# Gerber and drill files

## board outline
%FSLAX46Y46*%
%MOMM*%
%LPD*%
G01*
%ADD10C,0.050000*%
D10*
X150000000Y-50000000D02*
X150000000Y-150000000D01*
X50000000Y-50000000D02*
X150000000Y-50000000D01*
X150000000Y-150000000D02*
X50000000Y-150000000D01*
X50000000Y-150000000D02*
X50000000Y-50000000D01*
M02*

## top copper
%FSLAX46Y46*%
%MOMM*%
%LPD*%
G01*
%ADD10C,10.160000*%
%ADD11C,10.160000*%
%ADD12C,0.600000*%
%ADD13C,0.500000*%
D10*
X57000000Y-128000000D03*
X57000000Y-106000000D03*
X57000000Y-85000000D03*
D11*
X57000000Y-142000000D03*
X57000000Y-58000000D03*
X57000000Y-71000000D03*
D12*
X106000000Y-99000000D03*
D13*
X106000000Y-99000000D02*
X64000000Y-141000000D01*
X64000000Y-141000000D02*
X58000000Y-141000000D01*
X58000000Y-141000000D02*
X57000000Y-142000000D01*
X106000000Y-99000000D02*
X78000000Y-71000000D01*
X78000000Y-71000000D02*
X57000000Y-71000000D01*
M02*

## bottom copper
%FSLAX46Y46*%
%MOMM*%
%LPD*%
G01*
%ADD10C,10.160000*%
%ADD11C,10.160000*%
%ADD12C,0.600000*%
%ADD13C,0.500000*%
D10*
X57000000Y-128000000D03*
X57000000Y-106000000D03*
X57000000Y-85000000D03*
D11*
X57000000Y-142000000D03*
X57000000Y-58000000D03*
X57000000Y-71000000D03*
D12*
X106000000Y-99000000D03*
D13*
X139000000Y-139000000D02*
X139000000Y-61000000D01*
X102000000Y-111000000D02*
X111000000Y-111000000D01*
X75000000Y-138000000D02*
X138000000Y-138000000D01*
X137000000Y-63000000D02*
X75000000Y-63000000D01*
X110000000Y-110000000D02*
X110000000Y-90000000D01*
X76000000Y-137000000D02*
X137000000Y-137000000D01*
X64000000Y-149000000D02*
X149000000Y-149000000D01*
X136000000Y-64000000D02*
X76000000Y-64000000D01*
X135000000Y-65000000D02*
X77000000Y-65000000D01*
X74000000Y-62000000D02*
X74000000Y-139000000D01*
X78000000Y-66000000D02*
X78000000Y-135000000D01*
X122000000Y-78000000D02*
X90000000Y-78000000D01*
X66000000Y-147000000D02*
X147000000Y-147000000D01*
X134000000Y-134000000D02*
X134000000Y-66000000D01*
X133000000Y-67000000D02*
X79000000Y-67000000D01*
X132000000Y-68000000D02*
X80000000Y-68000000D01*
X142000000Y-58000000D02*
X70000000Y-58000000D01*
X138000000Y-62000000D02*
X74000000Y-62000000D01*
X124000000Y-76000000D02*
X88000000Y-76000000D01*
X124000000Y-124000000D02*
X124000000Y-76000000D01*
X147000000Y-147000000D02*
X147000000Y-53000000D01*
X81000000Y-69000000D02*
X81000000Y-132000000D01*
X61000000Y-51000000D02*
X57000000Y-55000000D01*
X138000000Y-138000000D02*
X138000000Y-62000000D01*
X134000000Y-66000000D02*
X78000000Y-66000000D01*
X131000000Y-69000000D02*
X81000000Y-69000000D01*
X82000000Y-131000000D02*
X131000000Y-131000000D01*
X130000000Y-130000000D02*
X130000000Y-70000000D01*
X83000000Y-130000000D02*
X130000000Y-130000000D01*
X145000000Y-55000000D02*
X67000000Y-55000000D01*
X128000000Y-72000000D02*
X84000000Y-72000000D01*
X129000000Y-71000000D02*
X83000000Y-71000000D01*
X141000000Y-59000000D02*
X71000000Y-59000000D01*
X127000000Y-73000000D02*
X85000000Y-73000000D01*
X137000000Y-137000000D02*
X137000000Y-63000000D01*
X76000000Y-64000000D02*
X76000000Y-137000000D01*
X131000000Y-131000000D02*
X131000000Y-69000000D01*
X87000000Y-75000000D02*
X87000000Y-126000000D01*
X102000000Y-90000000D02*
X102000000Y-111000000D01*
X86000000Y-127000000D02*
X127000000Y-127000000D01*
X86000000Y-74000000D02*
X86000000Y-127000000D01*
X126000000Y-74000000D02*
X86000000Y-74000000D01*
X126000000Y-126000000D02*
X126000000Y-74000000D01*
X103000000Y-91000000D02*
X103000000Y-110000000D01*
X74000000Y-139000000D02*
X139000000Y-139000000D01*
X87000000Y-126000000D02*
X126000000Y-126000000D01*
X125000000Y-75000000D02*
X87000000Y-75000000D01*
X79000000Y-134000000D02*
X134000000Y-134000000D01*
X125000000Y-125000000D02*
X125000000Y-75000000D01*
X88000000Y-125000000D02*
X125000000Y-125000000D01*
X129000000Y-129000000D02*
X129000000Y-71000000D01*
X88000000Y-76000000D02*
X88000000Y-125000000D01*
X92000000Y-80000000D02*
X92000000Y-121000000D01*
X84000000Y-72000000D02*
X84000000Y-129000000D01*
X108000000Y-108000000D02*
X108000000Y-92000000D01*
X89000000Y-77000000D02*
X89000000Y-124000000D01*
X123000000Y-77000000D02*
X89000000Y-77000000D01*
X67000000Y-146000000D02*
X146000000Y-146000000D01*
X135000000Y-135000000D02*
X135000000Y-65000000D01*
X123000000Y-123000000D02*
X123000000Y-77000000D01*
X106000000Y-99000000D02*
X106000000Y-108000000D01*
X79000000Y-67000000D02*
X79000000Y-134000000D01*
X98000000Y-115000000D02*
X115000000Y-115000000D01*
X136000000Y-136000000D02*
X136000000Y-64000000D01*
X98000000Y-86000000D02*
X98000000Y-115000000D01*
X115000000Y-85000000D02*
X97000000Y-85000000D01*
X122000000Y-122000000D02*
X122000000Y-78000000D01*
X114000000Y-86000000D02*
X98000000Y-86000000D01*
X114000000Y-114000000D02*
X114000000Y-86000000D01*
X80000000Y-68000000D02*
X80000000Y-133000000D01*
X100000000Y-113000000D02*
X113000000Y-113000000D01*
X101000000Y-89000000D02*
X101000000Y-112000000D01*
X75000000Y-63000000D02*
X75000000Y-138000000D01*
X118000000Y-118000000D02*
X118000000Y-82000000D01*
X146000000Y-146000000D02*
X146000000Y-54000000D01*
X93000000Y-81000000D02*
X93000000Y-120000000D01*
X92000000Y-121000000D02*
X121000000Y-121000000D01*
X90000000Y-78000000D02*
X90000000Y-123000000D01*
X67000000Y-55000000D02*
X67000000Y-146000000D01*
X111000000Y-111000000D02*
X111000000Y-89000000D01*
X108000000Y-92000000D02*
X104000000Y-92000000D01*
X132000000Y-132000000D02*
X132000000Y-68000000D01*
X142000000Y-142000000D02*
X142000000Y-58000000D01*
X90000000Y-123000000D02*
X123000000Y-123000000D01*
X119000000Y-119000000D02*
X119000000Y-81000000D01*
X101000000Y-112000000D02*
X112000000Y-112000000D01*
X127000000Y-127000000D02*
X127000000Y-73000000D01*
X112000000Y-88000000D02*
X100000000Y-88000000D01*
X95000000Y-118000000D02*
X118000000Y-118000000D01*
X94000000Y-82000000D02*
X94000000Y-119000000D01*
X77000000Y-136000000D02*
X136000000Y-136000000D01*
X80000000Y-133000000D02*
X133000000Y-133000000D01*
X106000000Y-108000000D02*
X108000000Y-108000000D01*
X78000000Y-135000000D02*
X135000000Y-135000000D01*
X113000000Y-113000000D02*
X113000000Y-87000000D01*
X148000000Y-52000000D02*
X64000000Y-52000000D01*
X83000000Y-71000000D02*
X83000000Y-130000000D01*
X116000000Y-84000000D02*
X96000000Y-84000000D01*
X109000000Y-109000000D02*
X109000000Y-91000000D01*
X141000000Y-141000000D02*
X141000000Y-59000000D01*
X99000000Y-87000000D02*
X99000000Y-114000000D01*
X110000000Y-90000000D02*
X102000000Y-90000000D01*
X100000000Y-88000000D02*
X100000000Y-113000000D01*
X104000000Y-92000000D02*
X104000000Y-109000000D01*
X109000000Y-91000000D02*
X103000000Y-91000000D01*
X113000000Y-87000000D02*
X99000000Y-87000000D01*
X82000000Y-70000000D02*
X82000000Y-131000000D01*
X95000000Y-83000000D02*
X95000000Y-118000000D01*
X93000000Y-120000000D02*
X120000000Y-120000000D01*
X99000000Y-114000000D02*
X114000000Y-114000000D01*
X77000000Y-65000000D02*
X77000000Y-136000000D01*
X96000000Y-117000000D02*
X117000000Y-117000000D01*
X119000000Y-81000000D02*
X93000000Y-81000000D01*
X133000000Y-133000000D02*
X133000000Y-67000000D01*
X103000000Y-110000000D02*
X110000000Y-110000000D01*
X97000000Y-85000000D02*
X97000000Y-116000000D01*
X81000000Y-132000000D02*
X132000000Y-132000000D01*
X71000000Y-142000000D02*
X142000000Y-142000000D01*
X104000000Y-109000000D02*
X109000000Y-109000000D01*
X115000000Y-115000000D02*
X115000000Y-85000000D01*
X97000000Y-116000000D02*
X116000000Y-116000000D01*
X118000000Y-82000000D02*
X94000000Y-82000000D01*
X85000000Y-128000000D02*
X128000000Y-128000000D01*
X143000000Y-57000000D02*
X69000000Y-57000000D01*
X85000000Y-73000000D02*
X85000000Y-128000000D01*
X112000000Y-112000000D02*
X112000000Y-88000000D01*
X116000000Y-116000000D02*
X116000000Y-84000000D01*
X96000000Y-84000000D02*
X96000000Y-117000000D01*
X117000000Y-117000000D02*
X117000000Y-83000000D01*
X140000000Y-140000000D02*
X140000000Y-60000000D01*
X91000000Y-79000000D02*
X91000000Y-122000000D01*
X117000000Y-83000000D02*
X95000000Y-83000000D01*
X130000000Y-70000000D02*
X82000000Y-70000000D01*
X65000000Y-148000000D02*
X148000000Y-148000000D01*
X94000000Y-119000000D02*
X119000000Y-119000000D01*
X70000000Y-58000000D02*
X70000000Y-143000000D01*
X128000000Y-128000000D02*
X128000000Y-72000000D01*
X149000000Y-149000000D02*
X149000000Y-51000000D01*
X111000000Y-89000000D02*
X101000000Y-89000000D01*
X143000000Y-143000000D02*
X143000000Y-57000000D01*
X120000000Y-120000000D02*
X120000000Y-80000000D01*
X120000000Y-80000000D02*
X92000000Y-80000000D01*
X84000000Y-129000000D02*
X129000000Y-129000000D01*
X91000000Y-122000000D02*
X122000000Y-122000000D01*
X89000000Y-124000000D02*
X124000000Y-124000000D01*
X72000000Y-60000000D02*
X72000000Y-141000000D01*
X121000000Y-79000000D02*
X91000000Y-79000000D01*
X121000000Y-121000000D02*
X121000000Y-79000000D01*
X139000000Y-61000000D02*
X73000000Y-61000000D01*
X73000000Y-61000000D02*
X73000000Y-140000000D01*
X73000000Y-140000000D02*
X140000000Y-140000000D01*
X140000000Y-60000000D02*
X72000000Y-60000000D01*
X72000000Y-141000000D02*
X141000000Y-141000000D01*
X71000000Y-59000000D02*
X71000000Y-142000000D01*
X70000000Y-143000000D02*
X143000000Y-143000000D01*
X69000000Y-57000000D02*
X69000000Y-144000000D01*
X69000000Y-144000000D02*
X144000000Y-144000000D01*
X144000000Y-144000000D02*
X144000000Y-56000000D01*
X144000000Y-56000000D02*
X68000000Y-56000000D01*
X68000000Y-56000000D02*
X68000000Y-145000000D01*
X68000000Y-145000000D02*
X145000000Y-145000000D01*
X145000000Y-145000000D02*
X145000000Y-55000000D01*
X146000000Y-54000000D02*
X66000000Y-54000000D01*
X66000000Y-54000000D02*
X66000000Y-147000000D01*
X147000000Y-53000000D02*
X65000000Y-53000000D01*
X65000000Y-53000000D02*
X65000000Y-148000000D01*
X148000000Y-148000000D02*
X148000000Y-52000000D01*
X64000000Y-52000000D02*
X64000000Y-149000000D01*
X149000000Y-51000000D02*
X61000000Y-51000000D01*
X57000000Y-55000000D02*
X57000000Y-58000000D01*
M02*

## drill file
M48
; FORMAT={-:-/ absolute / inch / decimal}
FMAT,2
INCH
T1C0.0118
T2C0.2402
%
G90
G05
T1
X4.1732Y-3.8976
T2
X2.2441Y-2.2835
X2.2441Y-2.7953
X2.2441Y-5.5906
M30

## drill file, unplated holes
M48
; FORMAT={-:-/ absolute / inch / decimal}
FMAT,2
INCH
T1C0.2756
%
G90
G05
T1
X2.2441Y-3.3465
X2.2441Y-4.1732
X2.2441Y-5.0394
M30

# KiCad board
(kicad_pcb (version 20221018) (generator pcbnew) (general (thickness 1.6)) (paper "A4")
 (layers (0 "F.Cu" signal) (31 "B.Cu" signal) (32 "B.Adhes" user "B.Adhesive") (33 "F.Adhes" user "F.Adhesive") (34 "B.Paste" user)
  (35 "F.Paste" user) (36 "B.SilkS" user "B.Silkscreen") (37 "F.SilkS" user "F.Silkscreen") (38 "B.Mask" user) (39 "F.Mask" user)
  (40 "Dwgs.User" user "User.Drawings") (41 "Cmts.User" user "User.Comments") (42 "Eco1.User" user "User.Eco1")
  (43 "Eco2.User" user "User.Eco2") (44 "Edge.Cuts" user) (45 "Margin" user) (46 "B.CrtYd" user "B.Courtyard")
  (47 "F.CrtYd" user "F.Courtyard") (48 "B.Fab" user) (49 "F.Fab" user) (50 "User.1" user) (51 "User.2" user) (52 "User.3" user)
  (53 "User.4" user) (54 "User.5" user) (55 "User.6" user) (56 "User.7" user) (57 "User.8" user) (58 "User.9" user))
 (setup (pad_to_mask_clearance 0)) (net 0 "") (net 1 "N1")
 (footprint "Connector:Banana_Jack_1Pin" (layer "F.Cu") (at 57 128)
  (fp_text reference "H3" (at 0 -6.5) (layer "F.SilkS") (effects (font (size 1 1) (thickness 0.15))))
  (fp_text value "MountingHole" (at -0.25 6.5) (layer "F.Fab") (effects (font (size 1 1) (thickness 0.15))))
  (pad "" np_thru_hole circle (at 0 0) (size 10.16 10.16) (drill 7) (layers "F&B.Cu" "*.Mask")))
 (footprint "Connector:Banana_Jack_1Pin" (layer "F.Cu") (at 57 58)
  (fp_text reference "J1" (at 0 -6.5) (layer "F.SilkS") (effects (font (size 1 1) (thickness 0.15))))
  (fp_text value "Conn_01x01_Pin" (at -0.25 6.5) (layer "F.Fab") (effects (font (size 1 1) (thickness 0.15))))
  (pad "1" thru_hole circle (at 0 0) (size 10.16 10.16) (drill 6.1) (layers "*.Cu" "*.Mask") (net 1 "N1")))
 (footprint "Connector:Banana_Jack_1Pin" (layer "F.Cu") (at 57 71)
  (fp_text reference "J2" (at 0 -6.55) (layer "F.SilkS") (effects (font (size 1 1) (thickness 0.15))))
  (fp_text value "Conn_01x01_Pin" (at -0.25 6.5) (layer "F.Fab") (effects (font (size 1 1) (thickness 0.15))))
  (pad "1" thru_hole circle (at 0 0) (size 10.16 10.16) (drill 6.1) (layers "*.Cu" "*.Mask") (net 1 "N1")))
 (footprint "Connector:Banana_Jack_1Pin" (layer "F.Cu") (at 57 106)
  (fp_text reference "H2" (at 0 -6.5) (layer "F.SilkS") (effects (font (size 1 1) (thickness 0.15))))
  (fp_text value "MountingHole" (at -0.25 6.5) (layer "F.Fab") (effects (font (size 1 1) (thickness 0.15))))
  (pad "" np_thru_hole circle (at 0 0) (size 10.16 10.16) (drill 7) (layers "F&B.Cu" "*.Mask")))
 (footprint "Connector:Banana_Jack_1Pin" (layer "F.Cu") (at 57 142)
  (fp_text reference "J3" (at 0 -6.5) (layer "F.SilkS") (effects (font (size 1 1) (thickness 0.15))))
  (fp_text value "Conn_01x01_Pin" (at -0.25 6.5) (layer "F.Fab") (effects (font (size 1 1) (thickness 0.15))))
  (pad "1" thru_hole circle (at 0 0) (size 10.16 10.16) (drill 6.1) (layers "*.Cu" "*.Mask") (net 1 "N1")))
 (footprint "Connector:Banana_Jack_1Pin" (layer "F.Cu") (at 57 85)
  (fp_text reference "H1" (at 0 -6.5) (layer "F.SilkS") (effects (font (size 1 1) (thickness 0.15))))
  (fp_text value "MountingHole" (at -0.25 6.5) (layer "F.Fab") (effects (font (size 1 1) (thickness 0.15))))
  (pad "" np_thru_hole circle (at 0 0) (size 10.16 10.16) (drill 7) (layers "F&B.Cu" "*.Mask")))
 (gr_line (start 150 50) (end 150 150) (stroke (width 0.05) (type default)) (layer "Edge.Cuts"))
 (gr_line (start 50 50) (end 150 50) (stroke (width 0.05) (type default)) (layer "Edge.Cuts"))
 (gr_line (start 150 150) (end 50 150) (stroke (width 0.05) (type default)) (layer "Edge.Cuts"))
 (gr_line (start 50 150) (end 50 50) (stroke (width 0.05) (type default)) (layer "Edge.Cuts"))
 (segment (start 106 99) (end 64 141) (width 0.5) (layer "F.Cu") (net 1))
 (segment (start 106 99) (end 78 71) (width 0.5) (layer "F.Cu") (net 1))
 (segment (start 64 141) (end 58 141) (width 0.5) (layer "F.Cu") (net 1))
 (segment (start 58 141) (end 57 142) (width 0.5) (layer "F.Cu") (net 1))
 (segment (start 78 71) (end 57 71) (width 0.5) (layer "F.Cu") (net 1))
 (via (at 106 99) (size 0.6) (drill 0.3) (layers "F.Cu" "B.Cu") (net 1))
 (segment (start 121 79) (end 91 79) (width 0.5) (layer "B.Cu") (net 1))
 (segment (start 82 131) (end 131 131) (width 0.5) (layer "B.Cu") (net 1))
 (segment (start 124 124) (end 124 76) (width 0.5) (layer "B.Cu") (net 1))
 (segment (start 83 71) (end 83 130) (width 0.5) (layer "B.Cu") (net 1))
 (segment (start 89 77) (end 89 124) (width 0.5) (layer "B.Cu") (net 1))
 (segment (start 100 113) (end 113 113) (width 0.5) (layer "B.Cu") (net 1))
 (segment (start 120 120) (end 120 80) (width 0.5) (layer "B.Cu") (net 1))
 (segment (start 67 146) (end 146 146) (width 0.5) (layer "B.Cu") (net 1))
 (segment (start 66 54) (end 66 147) (width 0.5) (layer "B.Cu") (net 1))
 (segment (start 92 80) (end 92 121) (width 0.5) (layer "B.Cu") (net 1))
 (segment (start 98 86) (end 98 115) (width 0.5) (layer "B.Cu") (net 1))
 (segment (start 90 123) (end 123 123) (width 0.5) (layer "B.Cu") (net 1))
 (segment (start 146 54) (end 66 54) (width 0.5) (layer "B.Cu") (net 1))
 (segment (start 120 80) (end 92 80) (width 0.5) (layer "B.Cu") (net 1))
 (segment (start 76 137) (end 137 137) (width 0.5) (layer "B.Cu") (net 1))
 (segment (start 92 121) (end 121 121) (width 0.5) (layer "B.Cu") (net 1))
 (segment (start 121 121) (end 121 79) (width 0.5) (layer "B.Cu") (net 1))
 (segment (start 112 88) (end 100 88) (width 0.5) (layer "B.Cu") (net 1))
 (segment (start 135 65) (end 77 65) (width 0.5) (layer "B.Cu") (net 1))
 (segment (start 68 145) (end 145 145) (width 0.5) (layer "B.Cu") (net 1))
 (segment (start 86 127) (end 127 127) (width 0.5) (layer "B.Cu") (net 1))
 (segment (start 73 140) (end 140 140) (width 0.5) (layer "B.Cu") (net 1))
 (segment (start 114 86) (end 98 86) (width 0.5) (layer "B.Cu") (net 1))
 (segment (start 96 117) (end 117 117) (width 0.5) (layer "B.Cu") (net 1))
 (segment (start 57 55) (end 57 58) (width 0.5) (layer "B.Cu") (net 1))
 (segment (start 95 118) (end 118 118) (width 0.5) (layer "B.Cu") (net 1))
 (segment (start 80 68) (end 80 133) (width 0.5) (layer "B.Cu") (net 1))
 (segment (start 83 130) (end 130 130) (width 0.5) (layer "B.Cu") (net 1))
 (segment (start 148 52) (end 64 52) (width 0.5) (layer "B.Cu") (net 1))
 (segment (start 145 145) (end 145 55) (width 0.5) (layer "B.Cu") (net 1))
 (segment (start 129 129) (end 129 71) (width 0.5) (layer "B.Cu") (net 1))
 (segment (start 68 56) (end 68 145) (width 0.5) (layer "B.Cu") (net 1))
 (segment (start 127 127) (end 127 73) (width 0.5) (layer "B.Cu") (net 1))
 (segment (start 109 91) (end 103 91) (width 0.5) (layer "B.Cu") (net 1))
 (segment (start 84 72) (end 84 129) (width 0.5) (layer "B.Cu") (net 1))
 (segment (start 71 59) (end 71 142) (width 0.5) (layer "B.Cu") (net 1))
 (segment (start 85 73) (end 85 128) (width 0.5) (layer "B.Cu") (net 1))
 (segment (start 102 90) (end 102 111) (width 0.5) (layer "B.Cu") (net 1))
 (segment (start 72 60) (end 72 141) (width 0.5) (layer "B.Cu") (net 1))
 (segment (start 142 142) (end 142 58) (width 0.5) (layer "B.Cu") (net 1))
 (segment (start 131 131) (end 131 69) (width 0.5) (layer "B.Cu") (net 1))
 (segment (start 65 148) (end 148 148) (width 0.5) (layer "B.Cu") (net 1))
 (segment (start 71 142) (end 142 142) (width 0.5) (layer "B.Cu") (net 1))
 (segment (start 101 89) (end 101 112) (width 0.5) (layer "B.Cu") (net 1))
 (segment (start 99 114) (end 114 114) (width 0.5) (layer "B.Cu") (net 1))
 (segment (start 149 51) (end 61 51) (width 0.5) (layer "B.Cu") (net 1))
 (segment (start 128 128) (end 128 72) (width 0.5) (layer "B.Cu") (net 1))
 (segment (start 72 141) (end 141 141) (width 0.5) (layer "B.Cu") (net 1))
 (segment (start 66 147) (end 147 147) (width 0.5) (layer "B.Cu") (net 1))
 (segment (start 126 74) (end 86 74) (width 0.5) (layer "B.Cu") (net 1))
 (segment (start 102 111) (end 111 111) (width 0.5) (layer "B.Cu") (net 1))
 (segment (start 87 126) (end 126 126) (width 0.5) (layer "B.Cu") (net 1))
 (segment (start 119 119) (end 119 81) (width 0.5) (layer "B.Cu") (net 1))
 (segment (start 133 67) (end 79 67) (width 0.5) (layer "B.Cu") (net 1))
 (segment (start 94 119) (end 119 119) (width 0.5) (layer "B.Cu") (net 1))
 (segment (start 90 78) (end 90 123) (width 0.5) (layer "B.Cu") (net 1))
 (segment (start 147 147) (end 147 53) (width 0.5) (layer "B.Cu") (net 1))
 (segment (start 146 146) (end 146 54) (width 0.5) (layer "B.Cu") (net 1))
 (segment (start 111 111) (end 111 89) (width 0.5) (layer "B.Cu") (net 1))
 (segment (start 74 62) (end 74 139) (width 0.5) (layer "B.Cu") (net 1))
 (segment (start 148 148) (end 148 52) (width 0.5) (layer "B.Cu") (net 1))
 (segment (start 147 53) (end 65 53) (width 0.5) (layer "B.Cu") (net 1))
 (segment (start 132 68) (end 80 68) (width 0.5) (layer "B.Cu") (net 1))
 (segment (start 79 67) (end 79 134) (width 0.5) (layer "B.Cu") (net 1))
 (segment (start 74 139) (end 139 139) (width 0.5) (layer "B.Cu") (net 1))
 (segment (start 125 125) (end 125 75) (width 0.5) (layer "B.Cu") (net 1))
 (segment (start 104 92) (end 104 109) (width 0.5) (layer "B.Cu") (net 1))
 (segment (start 125 75) (end 87 75) (width 0.5) (layer "B.Cu") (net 1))
 (segment (start 136 136) (end 136 64) (width 0.5) (layer "B.Cu") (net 1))
 (segment (start 61 51) (end 57 55) (width 0.5) (layer "B.Cu") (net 1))
 (segment (start 145 55) (end 67 55) (width 0.5) (layer "B.Cu") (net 1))
 (segment (start 113 87) (end 99 87) (width 0.5) (layer "B.Cu") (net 1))
 (segment (start 89 124) (end 124 124) (width 0.5) (layer "B.Cu") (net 1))
 (segment (start 129 71) (end 83 71) (width 0.5) (layer "B.Cu") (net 1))
 (segment (start 114 114) (end 114 86) (width 0.5) (layer "B.Cu") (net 1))
 (segment (start 85 128) (end 128 128) (width 0.5) (layer "B.Cu") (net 1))
 (segment (start 144 144) (end 144 56) (width 0.5) (layer "B.Cu") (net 1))
 (segment (start 97 116) (end 116 116) (width 0.5) (layer "B.Cu") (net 1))
 (segment (start 64 149) (end 149 149) (width 0.5) (layer "B.Cu") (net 1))
 (segment (start 139 61) (end 73 61) (width 0.5) (layer "B.Cu") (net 1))
 (segment (start 86 74) (end 86 127) (width 0.5) (layer "B.Cu") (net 1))
 (segment (start 93 81) (end 93 120) (width 0.5) (layer "B.Cu") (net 1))
 (segment (start 138 138) (end 138 62) (width 0.5) (layer "B.Cu") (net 1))
 (segment (start 118 118) (end 118 82) (width 0.5) (layer "B.Cu") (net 1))
 (segment (start 140 140) (end 140 60) (width 0.5) (layer "B.Cu") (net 1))
 (segment (start 106 99) (end 106 108) (width 0.5) (layer "B.Cu") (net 1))
 (segment (start 78 66) (end 78 135) (width 0.5) (layer "B.Cu") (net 1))
 (segment (start 138 62) (end 74 62) (width 0.5) (layer "B.Cu") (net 1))
 (segment (start 118 82) (end 94 82) (width 0.5) (layer "B.Cu") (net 1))
 (segment (start 110 90) (end 102 90) (width 0.5) (layer "B.Cu") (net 1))
 (segment (start 132 132) (end 132 68) (width 0.5) (layer "B.Cu") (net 1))
 (segment (start 78 135) (end 135 135) (width 0.5) (layer "B.Cu") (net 1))
 (segment (start 136 64) (end 76 64) (width 0.5) (layer "B.Cu") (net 1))
 (segment (start 75 63) (end 75 138) (width 0.5) (layer "B.Cu") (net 1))
 (segment (start 123 77) (end 89 77) (width 0.5) (layer "B.Cu") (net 1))
 (segment (start 134 66) (end 78 66) (width 0.5) (layer "B.Cu") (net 1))
 (segment (start 77 65) (end 77 136) (width 0.5) (layer "B.Cu") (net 1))
 (segment (start 141 59) (end 71 59) (width 0.5) (layer "B.Cu") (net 1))
 (segment (start 96 84) (end 96 117) (width 0.5) (layer "B.Cu") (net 1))
 (segment (start 135 135) (end 135 65) (width 0.5) (layer "B.Cu") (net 1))
 (segment (start 69 57) (end 69 144) (width 0.5) (layer "B.Cu") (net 1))
 (segment (start 143 143) (end 143 57) (width 0.5) (layer "B.Cu") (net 1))
 (segment (start 139 139) (end 139 61) (width 0.5) (layer "B.Cu") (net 1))
 (segment (start 76 64) (end 76 137) (width 0.5) (layer "B.Cu") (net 1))
 (segment (start 97 85) (end 97 116) (width 0.5) (layer "B.Cu") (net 1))
 (segment (start 116 84) (end 96 84) (width 0.5) (layer "B.Cu") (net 1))
 (segment (start 122 122) (end 122 78) (width 0.5) (layer "B.Cu") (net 1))
 (segment (start 144 56) (end 68 56) (width 0.5) (layer "B.Cu") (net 1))
 (segment (start 141 141) (end 141 59) (width 0.5) (layer "B.Cu") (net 1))
 (segment (start 101 112) (end 112 112) (width 0.5) (layer "B.Cu") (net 1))
 (segment (start 133 133) (end 133 67) (width 0.5) (layer "B.Cu") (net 1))
 (segment (start 69 144) (end 144 144) (width 0.5) (layer "B.Cu") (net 1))
 (segment (start 73 61) (end 73 140) (width 0.5) (layer "B.Cu") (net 1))
 (segment (start 88 76) (end 88 125) (width 0.5) (layer "B.Cu") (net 1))
 (segment (start 80 133) (end 133 133) (width 0.5) (layer "B.Cu") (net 1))
 (segment (start 127 73) (end 85 73) (width 0.5) (layer "B.Cu") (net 1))
 (segment (start 113 113) (end 113 87) (width 0.5) (layer "B.Cu") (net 1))
 (segment (start 142 58) (end 70 58) (width 0.5) (layer "B.Cu") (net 1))
 (segment (start 81 132) (end 132 132) (width 0.5) (layer "B.Cu") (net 1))
 (segment (start 104 109) (end 109 109) (width 0.5) (layer "B.Cu") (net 1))
 (segment (start 100 88) (end 100 113) (width 0.5) (layer "B.Cu") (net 1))
 (segment (start 82 70) (end 82 131) (width 0.5) (layer "B.Cu") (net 1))
 (segment (start 103 110) (end 110 110) (width 0.5) (layer "B.Cu") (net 1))
 (segment (start 115 115) (end 115 85) (width 0.5) (layer "B.Cu") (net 1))
 (segment (start 94 82) (end 94 119) (width 0.5) (layer "B.Cu") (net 1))
 (segment (start 110 110) (end 110 90) (width 0.5) (layer "B.Cu") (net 1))
 (segment (start 91 79) (end 91 122) (width 0.5) (layer "B.Cu") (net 1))
 (segment (start 140 60) (end 72 60) (width 0.5) (layer "B.Cu") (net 1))
 (segment (start 67 55) (end 67 146) (width 0.5) (layer "B.Cu") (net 1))
 (segment (start 70 58) (end 70 143) (width 0.5) (layer "B.Cu") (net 1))
 (segment (start 64 52) (end 64 149) (width 0.5) (layer "B.Cu") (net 1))
 (segment (start 137 137) (end 137 63) (width 0.5) (layer "B.Cu") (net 1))
 (segment (start 126 126) (end 126 74) (width 0.5) (layer "B.Cu") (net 1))
 (segment (start 130 70) (end 82 70) (width 0.5) (layer "B.Cu") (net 1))
 (segment (start 111 89) (end 101 89) (width 0.5) (layer "B.Cu") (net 1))
 (segment (start 98 115) (end 115 115) (width 0.5) (layer "B.Cu") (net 1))
 (segment (start 143 57) (end 69 57) (width 0.5) (layer "B.Cu") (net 1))
 (segment (start 81 69) (end 81 132) (width 0.5) (layer "B.Cu") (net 1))
 (segment (start 112 112) (end 112 88) (width 0.5) (layer "B.Cu") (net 1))
 (segment (start 99 87) (end 99 114) (width 0.5) (layer "B.Cu") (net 1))
 (segment (start 70 143) (end 143 143) (width 0.5) (layer "B.Cu") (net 1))
 (segment (start 103 91) (end 103 110) (width 0.5) (layer "B.Cu") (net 1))
 (segment (start 131 69) (end 81 69) (width 0.5) (layer "B.Cu") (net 1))
 (segment (start 95 83) (end 95 118) (width 0.5) (layer "B.Cu") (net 1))
 (segment (start 79 134) (end 134 134) (width 0.5) (layer "B.Cu") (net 1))
 (segment (start 149 149) (end 149 51) (width 0.5) (layer "B.Cu") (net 1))
 (segment (start 84 129) (end 129 129) (width 0.5) (layer "B.Cu") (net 1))
 (segment (start 137 63) (end 75 63) (width 0.5) (layer "B.Cu") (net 1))
 (segment (start 115 85) (end 97 85) (width 0.5) (layer "B.Cu") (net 1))
 (segment (start 134 134) (end 134 66) (width 0.5) (layer "B.Cu") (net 1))
 (segment (start 117 83) (end 95 83) (width 0.5) (layer "B.Cu") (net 1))
 (segment (start 75 138) (end 138 138) (width 0.5) (layer "B.Cu") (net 1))
 (segment (start 91 122) (end 122 122) (width 0.5) (layer "B.Cu") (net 1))
 (segment (start 124 76) (end 88 76) (width 0.5) (layer "B.Cu") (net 1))
 (segment (start 130 130) (end 130 70) (width 0.5) (layer "B.Cu") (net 1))
 (segment (start 108 92) (end 104 92) (width 0.5) (layer "B.Cu") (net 1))
 (segment (start 119 81) (end 93 81) (width 0.5) (layer "B.Cu") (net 1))
 (segment (start 128 72) (end 84 72) (width 0.5) (layer "B.Cu") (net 1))
 (segment (start 122 78) (end 90 78) (width 0.5) (layer "B.Cu") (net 1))
 (segment (start 117 117) (end 117 83) (width 0.5) (layer "B.Cu") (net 1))
 (segment (start 87 75) (end 87 126) (width 0.5) (layer "B.Cu") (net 1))
 (segment (start 123 123) (end 123 77) (width 0.5) (layer "B.Cu") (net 1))
 (segment (start 109 109) (end 109 91) (width 0.5) (layer "B.Cu") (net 1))
 (segment (start 65 53) (end 65 148) (width 0.5) (layer "B.Cu") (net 1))
 (segment (start 116 116) (end 116 84) (width 0.5) (layer "B.Cu") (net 1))
 (segment (start 108 108) (end 108 92) (width 0.5) (layer "B.Cu") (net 1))
 (segment (start 93 120) (end 120 120) (width 0.5) (layer "B.Cu") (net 1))
 (segment (start 77 136) (end 136 136) (width 0.5) (layer "B.Cu") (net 1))
 (segment (start 88 125) (end 125 125) (width 0.5) (layer "B.Cu") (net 1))
 (segment (start 106 108) (end 108 108) (width 0.5) (layer "B.Cu") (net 1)))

